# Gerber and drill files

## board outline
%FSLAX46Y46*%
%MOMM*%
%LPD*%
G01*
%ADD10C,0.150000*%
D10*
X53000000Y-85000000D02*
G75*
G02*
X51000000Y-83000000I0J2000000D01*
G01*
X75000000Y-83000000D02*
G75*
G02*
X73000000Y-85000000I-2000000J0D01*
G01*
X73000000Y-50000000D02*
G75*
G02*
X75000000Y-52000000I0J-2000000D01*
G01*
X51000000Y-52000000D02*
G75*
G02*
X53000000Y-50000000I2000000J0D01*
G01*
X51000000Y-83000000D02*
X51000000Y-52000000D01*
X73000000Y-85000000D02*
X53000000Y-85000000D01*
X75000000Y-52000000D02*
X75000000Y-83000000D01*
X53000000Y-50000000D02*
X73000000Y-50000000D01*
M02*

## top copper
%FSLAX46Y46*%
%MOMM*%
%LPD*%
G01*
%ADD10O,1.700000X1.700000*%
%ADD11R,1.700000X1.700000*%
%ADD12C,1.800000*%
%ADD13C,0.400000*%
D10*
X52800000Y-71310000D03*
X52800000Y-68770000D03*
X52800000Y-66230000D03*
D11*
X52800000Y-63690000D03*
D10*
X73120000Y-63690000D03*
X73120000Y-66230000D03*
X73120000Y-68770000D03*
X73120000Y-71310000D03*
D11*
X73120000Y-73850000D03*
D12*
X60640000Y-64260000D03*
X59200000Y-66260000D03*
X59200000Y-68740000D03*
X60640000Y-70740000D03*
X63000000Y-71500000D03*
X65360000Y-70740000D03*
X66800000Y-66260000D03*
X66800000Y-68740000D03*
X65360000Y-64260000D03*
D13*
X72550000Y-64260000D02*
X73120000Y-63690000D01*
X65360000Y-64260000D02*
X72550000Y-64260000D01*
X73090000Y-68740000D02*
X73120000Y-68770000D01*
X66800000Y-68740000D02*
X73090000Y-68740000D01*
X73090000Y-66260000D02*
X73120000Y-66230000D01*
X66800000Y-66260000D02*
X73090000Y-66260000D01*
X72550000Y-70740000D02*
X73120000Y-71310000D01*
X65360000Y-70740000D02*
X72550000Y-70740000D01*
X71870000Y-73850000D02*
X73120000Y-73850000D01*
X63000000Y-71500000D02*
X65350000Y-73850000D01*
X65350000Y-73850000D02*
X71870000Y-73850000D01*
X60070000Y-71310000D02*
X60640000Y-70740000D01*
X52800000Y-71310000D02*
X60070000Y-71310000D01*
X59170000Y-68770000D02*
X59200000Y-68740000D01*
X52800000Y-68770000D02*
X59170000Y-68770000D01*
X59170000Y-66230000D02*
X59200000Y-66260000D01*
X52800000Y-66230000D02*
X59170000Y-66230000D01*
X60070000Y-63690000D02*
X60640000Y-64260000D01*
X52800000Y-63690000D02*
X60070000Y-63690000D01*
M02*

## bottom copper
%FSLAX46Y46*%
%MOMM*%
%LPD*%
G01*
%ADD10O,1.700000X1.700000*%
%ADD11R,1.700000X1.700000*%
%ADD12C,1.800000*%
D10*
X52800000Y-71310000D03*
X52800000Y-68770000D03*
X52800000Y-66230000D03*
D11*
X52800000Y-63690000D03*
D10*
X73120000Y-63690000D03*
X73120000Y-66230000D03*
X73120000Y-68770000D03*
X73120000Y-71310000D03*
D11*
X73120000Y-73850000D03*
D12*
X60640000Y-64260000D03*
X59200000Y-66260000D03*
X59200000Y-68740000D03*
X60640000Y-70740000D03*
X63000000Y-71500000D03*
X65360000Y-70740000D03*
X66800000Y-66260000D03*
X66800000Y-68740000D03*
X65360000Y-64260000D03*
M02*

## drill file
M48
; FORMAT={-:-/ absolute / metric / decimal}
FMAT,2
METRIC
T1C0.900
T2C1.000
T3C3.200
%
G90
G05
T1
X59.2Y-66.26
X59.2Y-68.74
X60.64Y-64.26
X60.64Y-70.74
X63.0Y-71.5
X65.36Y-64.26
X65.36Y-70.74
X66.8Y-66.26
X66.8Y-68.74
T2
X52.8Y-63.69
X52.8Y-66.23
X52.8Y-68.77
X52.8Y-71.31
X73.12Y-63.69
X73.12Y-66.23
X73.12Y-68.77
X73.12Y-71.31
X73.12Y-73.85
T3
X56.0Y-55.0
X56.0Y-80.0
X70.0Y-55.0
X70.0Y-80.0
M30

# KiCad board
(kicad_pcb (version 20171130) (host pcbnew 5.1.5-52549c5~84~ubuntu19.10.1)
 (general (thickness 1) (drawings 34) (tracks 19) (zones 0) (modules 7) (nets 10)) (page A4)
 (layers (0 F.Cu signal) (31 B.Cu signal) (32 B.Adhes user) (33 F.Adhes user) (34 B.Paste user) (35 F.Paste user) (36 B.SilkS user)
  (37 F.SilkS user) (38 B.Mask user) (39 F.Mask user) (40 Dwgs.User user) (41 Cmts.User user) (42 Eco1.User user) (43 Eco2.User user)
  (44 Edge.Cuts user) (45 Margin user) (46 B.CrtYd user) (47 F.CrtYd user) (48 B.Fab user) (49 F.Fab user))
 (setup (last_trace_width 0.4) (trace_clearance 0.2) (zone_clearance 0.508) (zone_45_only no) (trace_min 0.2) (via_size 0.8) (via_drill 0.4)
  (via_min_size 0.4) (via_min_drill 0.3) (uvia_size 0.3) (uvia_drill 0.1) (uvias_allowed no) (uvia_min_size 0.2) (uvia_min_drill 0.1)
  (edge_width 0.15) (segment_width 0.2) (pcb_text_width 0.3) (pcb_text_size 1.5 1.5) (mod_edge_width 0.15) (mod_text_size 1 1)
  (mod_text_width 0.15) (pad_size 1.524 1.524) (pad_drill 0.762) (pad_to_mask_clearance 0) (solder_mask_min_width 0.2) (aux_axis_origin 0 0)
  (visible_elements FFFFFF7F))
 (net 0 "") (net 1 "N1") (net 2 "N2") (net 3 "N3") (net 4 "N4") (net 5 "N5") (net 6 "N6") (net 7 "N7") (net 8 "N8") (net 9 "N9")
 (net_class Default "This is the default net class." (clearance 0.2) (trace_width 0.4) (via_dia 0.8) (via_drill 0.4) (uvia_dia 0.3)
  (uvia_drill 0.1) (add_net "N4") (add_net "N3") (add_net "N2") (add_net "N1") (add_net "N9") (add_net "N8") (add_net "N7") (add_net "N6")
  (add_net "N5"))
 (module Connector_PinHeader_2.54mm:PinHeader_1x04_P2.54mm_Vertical (layer F.Cu) (at 52.8 63.69)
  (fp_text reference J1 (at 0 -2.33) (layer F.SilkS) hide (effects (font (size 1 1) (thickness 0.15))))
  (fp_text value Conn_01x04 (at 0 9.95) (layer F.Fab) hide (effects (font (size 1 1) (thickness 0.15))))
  (pad 4 thru_hole oval (at 0 7.62) (size 1.7 1.7) (drill 1) (layers *.Cu *.Mask) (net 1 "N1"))
  (pad 3 thru_hole oval (at 0 5.08) (size 1.7 1.7) (drill 1) (layers *.Cu *.Mask) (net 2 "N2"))
  (pad 2 thru_hole oval (at 0 2.54) (size 1.7 1.7) (drill 1) (layers *.Cu *.Mask) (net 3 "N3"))
  (pad 1 thru_hole rect (at 0 0) (size 1.7 1.7) (drill 1) (layers *.Cu *.Mask) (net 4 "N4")))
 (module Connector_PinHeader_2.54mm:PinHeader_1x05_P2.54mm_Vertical (layer F.Cu) (at 73.12 73.85 180)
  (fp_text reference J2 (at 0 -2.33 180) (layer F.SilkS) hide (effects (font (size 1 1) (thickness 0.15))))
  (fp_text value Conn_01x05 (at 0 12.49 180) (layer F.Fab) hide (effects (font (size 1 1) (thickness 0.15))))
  (pad 5 thru_hole oval (at 0 10.16 180) (size 1.7 1.7) (drill 1) (layers *.Cu *.Mask) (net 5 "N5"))
  (pad 4 thru_hole oval (at 0 7.62 180) (size 1.7 1.7) (drill 1) (layers *.Cu *.Mask) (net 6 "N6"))
  (pad 3 thru_hole oval (at 0 5.08 180) (size 1.7 1.7) (drill 1) (layers *.Cu *.Mask) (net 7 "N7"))
  (pad 2 thru_hole oval (at 0 2.54 180) (size 1.7 1.7) (drill 1) (layers *.Cu *.Mask) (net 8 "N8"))
  (pad 1 thru_hole rect (at 0 0 180) (size 1.7 1.7) (drill 1) (layers *.Cu *.Mask) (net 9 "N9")))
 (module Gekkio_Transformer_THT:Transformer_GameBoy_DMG (layer F.Cu) (at 63 67.5)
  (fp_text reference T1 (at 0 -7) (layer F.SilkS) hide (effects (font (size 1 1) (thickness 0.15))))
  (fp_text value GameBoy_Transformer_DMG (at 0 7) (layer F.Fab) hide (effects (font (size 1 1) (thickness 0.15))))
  (pad 1 thru_hole circle (at -2.36 -3.24 90) (size 1.8 1.8) (drill 0.9) (layers *.Cu *.Mask) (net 4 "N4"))
  (pad 2 thru_hole circle (at -3.8 -1.24 90) (size 1.8 1.8) (drill 0.9) (layers *.Cu *.Mask) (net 3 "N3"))
  (pad 3 thru_hole circle (at -3.8 1.24 90) (size 1.8 1.8) (drill 0.9) (layers *.Cu *.Mask) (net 2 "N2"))
  (pad 4 thru_hole circle (at -2.36 3.24 90) (size 1.8 1.8) (drill 0.9) (layers *.Cu *.Mask) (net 1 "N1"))
  (pad 5 thru_hole circle (at 0 4 90) (size 1.8 1.8) (drill 0.9) (layers *.Cu *.Mask) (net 9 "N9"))
  (pad 6 thru_hole circle (at 2.36 3.24 90) (size 1.8 1.8) (drill 0.9) (layers *.Cu *.Mask) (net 8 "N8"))
  (pad 8 thru_hole circle (at 3.8 -1.24 90) (size 1.8 1.8) (drill 0.9) (layers *.Cu *.Mask) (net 6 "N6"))
  (pad 7 thru_hole circle (at 3.8 1.24 90) (size 1.8 1.8) (drill 0.9) (layers *.Cu *.Mask) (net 7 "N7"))
  (pad 9 thru_hole circle (at 2.36 -3.24 90) (size 1.8 1.8) (drill 0.9) (layers *.Cu *.Mask) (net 5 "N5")))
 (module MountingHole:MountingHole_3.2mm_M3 (layer F.Cu) (at 70 80)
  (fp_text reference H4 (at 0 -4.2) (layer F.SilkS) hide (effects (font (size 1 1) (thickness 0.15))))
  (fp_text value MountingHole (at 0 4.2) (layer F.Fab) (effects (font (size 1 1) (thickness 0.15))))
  (pad 1 np_thru_hole circle (at 0 0) (size 3.2 3.2) (drill 3.2) (layers *.Cu *.Mask)))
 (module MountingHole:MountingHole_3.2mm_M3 (layer F.Cu) (at 56 80)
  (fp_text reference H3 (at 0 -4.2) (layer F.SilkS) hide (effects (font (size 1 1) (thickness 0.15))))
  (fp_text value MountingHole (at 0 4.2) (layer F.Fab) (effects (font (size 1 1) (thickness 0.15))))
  (pad 1 np_thru_hole circle (at 0 0) (size 3.2 3.2) (drill 3.2) (layers *.Cu *.Mask)))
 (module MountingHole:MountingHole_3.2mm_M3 (layer F.Cu) (at 70 55)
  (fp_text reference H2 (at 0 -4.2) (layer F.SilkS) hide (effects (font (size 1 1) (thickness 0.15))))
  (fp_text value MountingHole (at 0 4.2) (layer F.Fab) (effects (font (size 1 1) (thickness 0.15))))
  (pad 1 np_thru_hole circle (at 0 0) (size 3.2 3.2) (drill 3.2) (layers *.Cu *.Mask)))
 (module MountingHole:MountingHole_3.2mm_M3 (layer F.Cu) (at 56 55)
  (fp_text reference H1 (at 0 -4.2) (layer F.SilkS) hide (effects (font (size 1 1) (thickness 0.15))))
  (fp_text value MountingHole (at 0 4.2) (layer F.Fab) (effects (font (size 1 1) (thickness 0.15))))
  (pad 1 np_thru_hole circle (at 0 0) (size 3.2 3.2) (drill 3.2) (layers *.Cu *.Mask)))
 (gr_arc (start 53 83) (end 51 83) (angle -90) (layer Edge.Cuts) (width 0.15))
 (gr_arc (start 73 83) (end 73 85) (angle -90) (layer Edge.Cuts) (width 0.15))
 (gr_arc (start 73 52) (end 75 52) (angle -90) (layer Edge.Cuts) (width 0.15))
 (gr_arc (start 53 52) (end 53 50) (angle -90) (layer Edge.Cuts) (width 0.15))
 (gr_line (start 51 83) (end 51 52) (layer Edge.Cuts) (width 0.15))
 (gr_line (start 73 85) (end 53 85) (layer Edge.Cuts) (width 0.15))
 (gr_line (start 75 52) (end 75 83) (layer Edge.Cuts) (width 0.15))
 (gr_line (start 53 50) (end 73 50) (layer Edge.Cuts) (width 0.15))
 (segment (start 72.55 64.26) (end 73.12 63.69) (width 0.4) (layer F.Cu) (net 5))
 (segment (start 65.36 64.26) (end 72.55 64.26) (width 0.4) (layer F.Cu) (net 5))
 (segment (start 73.09 68.74) (end 73.12 68.77) (width 0.4) (layer F.Cu) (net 7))
 (segment (start 66.8 68.74) (end 73.09 68.74) (width 0.4) (layer F.Cu) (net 7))
 (segment (start 73.09 66.26) (end 73.12 66.23) (width 0.4) (layer F.Cu) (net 6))
 (segment (start 66.8 66.26) (end 73.09 66.26) (width 0.4) (layer F.Cu) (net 6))
 (segment (start 72.55 70.74) (end 73.12 71.31) (width 0.4) (layer F.Cu) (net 8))
 (segment (start 65.36 70.74) (end 72.55 70.74) (width 0.4) (layer F.Cu) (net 8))
 (segment (start 71.87 73.85) (end 73.12 73.85) (width 0.4) (layer F.Cu) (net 9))
 (segment (start 63 71.5) (end 65.35 73.85) (width 0.4) (layer F.Cu) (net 9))
 (segment (start 65.35 73.85) (end 71.87 73.85) (width 0.4) (layer F.Cu) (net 9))
 (segment (start 60.07 71.31) (end 60.64 70.74) (width 0.4) (layer F.Cu) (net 1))
 (segment (start 52.8 71.31) (end 60.07 71.31) (width 0.4) (layer F.Cu) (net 1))
 (segment (start 59.17 68.77) (end 59.2 68.74) (width 0.4) (layer F.Cu) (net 2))
 (segment (start 52.8 68.77) (end 59.17 68.77) (width 0.4) (layer F.Cu) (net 2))
 (segment (start 59.17 66.23) (end 59.2 66.26) (width 0.4) (layer F.Cu) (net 3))
 (segment (start 52.8 66.23) (end 59.17 66.23) (width 0.4) (layer F.Cu) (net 3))
 (segment (start 60.07 63.69) (end 60.64 64.26) (width 0.4) (layer F.Cu) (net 4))
 (segment (start 52.8 63.69) (end 60.07 63.69) (width 0.4) (layer F.Cu) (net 4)))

